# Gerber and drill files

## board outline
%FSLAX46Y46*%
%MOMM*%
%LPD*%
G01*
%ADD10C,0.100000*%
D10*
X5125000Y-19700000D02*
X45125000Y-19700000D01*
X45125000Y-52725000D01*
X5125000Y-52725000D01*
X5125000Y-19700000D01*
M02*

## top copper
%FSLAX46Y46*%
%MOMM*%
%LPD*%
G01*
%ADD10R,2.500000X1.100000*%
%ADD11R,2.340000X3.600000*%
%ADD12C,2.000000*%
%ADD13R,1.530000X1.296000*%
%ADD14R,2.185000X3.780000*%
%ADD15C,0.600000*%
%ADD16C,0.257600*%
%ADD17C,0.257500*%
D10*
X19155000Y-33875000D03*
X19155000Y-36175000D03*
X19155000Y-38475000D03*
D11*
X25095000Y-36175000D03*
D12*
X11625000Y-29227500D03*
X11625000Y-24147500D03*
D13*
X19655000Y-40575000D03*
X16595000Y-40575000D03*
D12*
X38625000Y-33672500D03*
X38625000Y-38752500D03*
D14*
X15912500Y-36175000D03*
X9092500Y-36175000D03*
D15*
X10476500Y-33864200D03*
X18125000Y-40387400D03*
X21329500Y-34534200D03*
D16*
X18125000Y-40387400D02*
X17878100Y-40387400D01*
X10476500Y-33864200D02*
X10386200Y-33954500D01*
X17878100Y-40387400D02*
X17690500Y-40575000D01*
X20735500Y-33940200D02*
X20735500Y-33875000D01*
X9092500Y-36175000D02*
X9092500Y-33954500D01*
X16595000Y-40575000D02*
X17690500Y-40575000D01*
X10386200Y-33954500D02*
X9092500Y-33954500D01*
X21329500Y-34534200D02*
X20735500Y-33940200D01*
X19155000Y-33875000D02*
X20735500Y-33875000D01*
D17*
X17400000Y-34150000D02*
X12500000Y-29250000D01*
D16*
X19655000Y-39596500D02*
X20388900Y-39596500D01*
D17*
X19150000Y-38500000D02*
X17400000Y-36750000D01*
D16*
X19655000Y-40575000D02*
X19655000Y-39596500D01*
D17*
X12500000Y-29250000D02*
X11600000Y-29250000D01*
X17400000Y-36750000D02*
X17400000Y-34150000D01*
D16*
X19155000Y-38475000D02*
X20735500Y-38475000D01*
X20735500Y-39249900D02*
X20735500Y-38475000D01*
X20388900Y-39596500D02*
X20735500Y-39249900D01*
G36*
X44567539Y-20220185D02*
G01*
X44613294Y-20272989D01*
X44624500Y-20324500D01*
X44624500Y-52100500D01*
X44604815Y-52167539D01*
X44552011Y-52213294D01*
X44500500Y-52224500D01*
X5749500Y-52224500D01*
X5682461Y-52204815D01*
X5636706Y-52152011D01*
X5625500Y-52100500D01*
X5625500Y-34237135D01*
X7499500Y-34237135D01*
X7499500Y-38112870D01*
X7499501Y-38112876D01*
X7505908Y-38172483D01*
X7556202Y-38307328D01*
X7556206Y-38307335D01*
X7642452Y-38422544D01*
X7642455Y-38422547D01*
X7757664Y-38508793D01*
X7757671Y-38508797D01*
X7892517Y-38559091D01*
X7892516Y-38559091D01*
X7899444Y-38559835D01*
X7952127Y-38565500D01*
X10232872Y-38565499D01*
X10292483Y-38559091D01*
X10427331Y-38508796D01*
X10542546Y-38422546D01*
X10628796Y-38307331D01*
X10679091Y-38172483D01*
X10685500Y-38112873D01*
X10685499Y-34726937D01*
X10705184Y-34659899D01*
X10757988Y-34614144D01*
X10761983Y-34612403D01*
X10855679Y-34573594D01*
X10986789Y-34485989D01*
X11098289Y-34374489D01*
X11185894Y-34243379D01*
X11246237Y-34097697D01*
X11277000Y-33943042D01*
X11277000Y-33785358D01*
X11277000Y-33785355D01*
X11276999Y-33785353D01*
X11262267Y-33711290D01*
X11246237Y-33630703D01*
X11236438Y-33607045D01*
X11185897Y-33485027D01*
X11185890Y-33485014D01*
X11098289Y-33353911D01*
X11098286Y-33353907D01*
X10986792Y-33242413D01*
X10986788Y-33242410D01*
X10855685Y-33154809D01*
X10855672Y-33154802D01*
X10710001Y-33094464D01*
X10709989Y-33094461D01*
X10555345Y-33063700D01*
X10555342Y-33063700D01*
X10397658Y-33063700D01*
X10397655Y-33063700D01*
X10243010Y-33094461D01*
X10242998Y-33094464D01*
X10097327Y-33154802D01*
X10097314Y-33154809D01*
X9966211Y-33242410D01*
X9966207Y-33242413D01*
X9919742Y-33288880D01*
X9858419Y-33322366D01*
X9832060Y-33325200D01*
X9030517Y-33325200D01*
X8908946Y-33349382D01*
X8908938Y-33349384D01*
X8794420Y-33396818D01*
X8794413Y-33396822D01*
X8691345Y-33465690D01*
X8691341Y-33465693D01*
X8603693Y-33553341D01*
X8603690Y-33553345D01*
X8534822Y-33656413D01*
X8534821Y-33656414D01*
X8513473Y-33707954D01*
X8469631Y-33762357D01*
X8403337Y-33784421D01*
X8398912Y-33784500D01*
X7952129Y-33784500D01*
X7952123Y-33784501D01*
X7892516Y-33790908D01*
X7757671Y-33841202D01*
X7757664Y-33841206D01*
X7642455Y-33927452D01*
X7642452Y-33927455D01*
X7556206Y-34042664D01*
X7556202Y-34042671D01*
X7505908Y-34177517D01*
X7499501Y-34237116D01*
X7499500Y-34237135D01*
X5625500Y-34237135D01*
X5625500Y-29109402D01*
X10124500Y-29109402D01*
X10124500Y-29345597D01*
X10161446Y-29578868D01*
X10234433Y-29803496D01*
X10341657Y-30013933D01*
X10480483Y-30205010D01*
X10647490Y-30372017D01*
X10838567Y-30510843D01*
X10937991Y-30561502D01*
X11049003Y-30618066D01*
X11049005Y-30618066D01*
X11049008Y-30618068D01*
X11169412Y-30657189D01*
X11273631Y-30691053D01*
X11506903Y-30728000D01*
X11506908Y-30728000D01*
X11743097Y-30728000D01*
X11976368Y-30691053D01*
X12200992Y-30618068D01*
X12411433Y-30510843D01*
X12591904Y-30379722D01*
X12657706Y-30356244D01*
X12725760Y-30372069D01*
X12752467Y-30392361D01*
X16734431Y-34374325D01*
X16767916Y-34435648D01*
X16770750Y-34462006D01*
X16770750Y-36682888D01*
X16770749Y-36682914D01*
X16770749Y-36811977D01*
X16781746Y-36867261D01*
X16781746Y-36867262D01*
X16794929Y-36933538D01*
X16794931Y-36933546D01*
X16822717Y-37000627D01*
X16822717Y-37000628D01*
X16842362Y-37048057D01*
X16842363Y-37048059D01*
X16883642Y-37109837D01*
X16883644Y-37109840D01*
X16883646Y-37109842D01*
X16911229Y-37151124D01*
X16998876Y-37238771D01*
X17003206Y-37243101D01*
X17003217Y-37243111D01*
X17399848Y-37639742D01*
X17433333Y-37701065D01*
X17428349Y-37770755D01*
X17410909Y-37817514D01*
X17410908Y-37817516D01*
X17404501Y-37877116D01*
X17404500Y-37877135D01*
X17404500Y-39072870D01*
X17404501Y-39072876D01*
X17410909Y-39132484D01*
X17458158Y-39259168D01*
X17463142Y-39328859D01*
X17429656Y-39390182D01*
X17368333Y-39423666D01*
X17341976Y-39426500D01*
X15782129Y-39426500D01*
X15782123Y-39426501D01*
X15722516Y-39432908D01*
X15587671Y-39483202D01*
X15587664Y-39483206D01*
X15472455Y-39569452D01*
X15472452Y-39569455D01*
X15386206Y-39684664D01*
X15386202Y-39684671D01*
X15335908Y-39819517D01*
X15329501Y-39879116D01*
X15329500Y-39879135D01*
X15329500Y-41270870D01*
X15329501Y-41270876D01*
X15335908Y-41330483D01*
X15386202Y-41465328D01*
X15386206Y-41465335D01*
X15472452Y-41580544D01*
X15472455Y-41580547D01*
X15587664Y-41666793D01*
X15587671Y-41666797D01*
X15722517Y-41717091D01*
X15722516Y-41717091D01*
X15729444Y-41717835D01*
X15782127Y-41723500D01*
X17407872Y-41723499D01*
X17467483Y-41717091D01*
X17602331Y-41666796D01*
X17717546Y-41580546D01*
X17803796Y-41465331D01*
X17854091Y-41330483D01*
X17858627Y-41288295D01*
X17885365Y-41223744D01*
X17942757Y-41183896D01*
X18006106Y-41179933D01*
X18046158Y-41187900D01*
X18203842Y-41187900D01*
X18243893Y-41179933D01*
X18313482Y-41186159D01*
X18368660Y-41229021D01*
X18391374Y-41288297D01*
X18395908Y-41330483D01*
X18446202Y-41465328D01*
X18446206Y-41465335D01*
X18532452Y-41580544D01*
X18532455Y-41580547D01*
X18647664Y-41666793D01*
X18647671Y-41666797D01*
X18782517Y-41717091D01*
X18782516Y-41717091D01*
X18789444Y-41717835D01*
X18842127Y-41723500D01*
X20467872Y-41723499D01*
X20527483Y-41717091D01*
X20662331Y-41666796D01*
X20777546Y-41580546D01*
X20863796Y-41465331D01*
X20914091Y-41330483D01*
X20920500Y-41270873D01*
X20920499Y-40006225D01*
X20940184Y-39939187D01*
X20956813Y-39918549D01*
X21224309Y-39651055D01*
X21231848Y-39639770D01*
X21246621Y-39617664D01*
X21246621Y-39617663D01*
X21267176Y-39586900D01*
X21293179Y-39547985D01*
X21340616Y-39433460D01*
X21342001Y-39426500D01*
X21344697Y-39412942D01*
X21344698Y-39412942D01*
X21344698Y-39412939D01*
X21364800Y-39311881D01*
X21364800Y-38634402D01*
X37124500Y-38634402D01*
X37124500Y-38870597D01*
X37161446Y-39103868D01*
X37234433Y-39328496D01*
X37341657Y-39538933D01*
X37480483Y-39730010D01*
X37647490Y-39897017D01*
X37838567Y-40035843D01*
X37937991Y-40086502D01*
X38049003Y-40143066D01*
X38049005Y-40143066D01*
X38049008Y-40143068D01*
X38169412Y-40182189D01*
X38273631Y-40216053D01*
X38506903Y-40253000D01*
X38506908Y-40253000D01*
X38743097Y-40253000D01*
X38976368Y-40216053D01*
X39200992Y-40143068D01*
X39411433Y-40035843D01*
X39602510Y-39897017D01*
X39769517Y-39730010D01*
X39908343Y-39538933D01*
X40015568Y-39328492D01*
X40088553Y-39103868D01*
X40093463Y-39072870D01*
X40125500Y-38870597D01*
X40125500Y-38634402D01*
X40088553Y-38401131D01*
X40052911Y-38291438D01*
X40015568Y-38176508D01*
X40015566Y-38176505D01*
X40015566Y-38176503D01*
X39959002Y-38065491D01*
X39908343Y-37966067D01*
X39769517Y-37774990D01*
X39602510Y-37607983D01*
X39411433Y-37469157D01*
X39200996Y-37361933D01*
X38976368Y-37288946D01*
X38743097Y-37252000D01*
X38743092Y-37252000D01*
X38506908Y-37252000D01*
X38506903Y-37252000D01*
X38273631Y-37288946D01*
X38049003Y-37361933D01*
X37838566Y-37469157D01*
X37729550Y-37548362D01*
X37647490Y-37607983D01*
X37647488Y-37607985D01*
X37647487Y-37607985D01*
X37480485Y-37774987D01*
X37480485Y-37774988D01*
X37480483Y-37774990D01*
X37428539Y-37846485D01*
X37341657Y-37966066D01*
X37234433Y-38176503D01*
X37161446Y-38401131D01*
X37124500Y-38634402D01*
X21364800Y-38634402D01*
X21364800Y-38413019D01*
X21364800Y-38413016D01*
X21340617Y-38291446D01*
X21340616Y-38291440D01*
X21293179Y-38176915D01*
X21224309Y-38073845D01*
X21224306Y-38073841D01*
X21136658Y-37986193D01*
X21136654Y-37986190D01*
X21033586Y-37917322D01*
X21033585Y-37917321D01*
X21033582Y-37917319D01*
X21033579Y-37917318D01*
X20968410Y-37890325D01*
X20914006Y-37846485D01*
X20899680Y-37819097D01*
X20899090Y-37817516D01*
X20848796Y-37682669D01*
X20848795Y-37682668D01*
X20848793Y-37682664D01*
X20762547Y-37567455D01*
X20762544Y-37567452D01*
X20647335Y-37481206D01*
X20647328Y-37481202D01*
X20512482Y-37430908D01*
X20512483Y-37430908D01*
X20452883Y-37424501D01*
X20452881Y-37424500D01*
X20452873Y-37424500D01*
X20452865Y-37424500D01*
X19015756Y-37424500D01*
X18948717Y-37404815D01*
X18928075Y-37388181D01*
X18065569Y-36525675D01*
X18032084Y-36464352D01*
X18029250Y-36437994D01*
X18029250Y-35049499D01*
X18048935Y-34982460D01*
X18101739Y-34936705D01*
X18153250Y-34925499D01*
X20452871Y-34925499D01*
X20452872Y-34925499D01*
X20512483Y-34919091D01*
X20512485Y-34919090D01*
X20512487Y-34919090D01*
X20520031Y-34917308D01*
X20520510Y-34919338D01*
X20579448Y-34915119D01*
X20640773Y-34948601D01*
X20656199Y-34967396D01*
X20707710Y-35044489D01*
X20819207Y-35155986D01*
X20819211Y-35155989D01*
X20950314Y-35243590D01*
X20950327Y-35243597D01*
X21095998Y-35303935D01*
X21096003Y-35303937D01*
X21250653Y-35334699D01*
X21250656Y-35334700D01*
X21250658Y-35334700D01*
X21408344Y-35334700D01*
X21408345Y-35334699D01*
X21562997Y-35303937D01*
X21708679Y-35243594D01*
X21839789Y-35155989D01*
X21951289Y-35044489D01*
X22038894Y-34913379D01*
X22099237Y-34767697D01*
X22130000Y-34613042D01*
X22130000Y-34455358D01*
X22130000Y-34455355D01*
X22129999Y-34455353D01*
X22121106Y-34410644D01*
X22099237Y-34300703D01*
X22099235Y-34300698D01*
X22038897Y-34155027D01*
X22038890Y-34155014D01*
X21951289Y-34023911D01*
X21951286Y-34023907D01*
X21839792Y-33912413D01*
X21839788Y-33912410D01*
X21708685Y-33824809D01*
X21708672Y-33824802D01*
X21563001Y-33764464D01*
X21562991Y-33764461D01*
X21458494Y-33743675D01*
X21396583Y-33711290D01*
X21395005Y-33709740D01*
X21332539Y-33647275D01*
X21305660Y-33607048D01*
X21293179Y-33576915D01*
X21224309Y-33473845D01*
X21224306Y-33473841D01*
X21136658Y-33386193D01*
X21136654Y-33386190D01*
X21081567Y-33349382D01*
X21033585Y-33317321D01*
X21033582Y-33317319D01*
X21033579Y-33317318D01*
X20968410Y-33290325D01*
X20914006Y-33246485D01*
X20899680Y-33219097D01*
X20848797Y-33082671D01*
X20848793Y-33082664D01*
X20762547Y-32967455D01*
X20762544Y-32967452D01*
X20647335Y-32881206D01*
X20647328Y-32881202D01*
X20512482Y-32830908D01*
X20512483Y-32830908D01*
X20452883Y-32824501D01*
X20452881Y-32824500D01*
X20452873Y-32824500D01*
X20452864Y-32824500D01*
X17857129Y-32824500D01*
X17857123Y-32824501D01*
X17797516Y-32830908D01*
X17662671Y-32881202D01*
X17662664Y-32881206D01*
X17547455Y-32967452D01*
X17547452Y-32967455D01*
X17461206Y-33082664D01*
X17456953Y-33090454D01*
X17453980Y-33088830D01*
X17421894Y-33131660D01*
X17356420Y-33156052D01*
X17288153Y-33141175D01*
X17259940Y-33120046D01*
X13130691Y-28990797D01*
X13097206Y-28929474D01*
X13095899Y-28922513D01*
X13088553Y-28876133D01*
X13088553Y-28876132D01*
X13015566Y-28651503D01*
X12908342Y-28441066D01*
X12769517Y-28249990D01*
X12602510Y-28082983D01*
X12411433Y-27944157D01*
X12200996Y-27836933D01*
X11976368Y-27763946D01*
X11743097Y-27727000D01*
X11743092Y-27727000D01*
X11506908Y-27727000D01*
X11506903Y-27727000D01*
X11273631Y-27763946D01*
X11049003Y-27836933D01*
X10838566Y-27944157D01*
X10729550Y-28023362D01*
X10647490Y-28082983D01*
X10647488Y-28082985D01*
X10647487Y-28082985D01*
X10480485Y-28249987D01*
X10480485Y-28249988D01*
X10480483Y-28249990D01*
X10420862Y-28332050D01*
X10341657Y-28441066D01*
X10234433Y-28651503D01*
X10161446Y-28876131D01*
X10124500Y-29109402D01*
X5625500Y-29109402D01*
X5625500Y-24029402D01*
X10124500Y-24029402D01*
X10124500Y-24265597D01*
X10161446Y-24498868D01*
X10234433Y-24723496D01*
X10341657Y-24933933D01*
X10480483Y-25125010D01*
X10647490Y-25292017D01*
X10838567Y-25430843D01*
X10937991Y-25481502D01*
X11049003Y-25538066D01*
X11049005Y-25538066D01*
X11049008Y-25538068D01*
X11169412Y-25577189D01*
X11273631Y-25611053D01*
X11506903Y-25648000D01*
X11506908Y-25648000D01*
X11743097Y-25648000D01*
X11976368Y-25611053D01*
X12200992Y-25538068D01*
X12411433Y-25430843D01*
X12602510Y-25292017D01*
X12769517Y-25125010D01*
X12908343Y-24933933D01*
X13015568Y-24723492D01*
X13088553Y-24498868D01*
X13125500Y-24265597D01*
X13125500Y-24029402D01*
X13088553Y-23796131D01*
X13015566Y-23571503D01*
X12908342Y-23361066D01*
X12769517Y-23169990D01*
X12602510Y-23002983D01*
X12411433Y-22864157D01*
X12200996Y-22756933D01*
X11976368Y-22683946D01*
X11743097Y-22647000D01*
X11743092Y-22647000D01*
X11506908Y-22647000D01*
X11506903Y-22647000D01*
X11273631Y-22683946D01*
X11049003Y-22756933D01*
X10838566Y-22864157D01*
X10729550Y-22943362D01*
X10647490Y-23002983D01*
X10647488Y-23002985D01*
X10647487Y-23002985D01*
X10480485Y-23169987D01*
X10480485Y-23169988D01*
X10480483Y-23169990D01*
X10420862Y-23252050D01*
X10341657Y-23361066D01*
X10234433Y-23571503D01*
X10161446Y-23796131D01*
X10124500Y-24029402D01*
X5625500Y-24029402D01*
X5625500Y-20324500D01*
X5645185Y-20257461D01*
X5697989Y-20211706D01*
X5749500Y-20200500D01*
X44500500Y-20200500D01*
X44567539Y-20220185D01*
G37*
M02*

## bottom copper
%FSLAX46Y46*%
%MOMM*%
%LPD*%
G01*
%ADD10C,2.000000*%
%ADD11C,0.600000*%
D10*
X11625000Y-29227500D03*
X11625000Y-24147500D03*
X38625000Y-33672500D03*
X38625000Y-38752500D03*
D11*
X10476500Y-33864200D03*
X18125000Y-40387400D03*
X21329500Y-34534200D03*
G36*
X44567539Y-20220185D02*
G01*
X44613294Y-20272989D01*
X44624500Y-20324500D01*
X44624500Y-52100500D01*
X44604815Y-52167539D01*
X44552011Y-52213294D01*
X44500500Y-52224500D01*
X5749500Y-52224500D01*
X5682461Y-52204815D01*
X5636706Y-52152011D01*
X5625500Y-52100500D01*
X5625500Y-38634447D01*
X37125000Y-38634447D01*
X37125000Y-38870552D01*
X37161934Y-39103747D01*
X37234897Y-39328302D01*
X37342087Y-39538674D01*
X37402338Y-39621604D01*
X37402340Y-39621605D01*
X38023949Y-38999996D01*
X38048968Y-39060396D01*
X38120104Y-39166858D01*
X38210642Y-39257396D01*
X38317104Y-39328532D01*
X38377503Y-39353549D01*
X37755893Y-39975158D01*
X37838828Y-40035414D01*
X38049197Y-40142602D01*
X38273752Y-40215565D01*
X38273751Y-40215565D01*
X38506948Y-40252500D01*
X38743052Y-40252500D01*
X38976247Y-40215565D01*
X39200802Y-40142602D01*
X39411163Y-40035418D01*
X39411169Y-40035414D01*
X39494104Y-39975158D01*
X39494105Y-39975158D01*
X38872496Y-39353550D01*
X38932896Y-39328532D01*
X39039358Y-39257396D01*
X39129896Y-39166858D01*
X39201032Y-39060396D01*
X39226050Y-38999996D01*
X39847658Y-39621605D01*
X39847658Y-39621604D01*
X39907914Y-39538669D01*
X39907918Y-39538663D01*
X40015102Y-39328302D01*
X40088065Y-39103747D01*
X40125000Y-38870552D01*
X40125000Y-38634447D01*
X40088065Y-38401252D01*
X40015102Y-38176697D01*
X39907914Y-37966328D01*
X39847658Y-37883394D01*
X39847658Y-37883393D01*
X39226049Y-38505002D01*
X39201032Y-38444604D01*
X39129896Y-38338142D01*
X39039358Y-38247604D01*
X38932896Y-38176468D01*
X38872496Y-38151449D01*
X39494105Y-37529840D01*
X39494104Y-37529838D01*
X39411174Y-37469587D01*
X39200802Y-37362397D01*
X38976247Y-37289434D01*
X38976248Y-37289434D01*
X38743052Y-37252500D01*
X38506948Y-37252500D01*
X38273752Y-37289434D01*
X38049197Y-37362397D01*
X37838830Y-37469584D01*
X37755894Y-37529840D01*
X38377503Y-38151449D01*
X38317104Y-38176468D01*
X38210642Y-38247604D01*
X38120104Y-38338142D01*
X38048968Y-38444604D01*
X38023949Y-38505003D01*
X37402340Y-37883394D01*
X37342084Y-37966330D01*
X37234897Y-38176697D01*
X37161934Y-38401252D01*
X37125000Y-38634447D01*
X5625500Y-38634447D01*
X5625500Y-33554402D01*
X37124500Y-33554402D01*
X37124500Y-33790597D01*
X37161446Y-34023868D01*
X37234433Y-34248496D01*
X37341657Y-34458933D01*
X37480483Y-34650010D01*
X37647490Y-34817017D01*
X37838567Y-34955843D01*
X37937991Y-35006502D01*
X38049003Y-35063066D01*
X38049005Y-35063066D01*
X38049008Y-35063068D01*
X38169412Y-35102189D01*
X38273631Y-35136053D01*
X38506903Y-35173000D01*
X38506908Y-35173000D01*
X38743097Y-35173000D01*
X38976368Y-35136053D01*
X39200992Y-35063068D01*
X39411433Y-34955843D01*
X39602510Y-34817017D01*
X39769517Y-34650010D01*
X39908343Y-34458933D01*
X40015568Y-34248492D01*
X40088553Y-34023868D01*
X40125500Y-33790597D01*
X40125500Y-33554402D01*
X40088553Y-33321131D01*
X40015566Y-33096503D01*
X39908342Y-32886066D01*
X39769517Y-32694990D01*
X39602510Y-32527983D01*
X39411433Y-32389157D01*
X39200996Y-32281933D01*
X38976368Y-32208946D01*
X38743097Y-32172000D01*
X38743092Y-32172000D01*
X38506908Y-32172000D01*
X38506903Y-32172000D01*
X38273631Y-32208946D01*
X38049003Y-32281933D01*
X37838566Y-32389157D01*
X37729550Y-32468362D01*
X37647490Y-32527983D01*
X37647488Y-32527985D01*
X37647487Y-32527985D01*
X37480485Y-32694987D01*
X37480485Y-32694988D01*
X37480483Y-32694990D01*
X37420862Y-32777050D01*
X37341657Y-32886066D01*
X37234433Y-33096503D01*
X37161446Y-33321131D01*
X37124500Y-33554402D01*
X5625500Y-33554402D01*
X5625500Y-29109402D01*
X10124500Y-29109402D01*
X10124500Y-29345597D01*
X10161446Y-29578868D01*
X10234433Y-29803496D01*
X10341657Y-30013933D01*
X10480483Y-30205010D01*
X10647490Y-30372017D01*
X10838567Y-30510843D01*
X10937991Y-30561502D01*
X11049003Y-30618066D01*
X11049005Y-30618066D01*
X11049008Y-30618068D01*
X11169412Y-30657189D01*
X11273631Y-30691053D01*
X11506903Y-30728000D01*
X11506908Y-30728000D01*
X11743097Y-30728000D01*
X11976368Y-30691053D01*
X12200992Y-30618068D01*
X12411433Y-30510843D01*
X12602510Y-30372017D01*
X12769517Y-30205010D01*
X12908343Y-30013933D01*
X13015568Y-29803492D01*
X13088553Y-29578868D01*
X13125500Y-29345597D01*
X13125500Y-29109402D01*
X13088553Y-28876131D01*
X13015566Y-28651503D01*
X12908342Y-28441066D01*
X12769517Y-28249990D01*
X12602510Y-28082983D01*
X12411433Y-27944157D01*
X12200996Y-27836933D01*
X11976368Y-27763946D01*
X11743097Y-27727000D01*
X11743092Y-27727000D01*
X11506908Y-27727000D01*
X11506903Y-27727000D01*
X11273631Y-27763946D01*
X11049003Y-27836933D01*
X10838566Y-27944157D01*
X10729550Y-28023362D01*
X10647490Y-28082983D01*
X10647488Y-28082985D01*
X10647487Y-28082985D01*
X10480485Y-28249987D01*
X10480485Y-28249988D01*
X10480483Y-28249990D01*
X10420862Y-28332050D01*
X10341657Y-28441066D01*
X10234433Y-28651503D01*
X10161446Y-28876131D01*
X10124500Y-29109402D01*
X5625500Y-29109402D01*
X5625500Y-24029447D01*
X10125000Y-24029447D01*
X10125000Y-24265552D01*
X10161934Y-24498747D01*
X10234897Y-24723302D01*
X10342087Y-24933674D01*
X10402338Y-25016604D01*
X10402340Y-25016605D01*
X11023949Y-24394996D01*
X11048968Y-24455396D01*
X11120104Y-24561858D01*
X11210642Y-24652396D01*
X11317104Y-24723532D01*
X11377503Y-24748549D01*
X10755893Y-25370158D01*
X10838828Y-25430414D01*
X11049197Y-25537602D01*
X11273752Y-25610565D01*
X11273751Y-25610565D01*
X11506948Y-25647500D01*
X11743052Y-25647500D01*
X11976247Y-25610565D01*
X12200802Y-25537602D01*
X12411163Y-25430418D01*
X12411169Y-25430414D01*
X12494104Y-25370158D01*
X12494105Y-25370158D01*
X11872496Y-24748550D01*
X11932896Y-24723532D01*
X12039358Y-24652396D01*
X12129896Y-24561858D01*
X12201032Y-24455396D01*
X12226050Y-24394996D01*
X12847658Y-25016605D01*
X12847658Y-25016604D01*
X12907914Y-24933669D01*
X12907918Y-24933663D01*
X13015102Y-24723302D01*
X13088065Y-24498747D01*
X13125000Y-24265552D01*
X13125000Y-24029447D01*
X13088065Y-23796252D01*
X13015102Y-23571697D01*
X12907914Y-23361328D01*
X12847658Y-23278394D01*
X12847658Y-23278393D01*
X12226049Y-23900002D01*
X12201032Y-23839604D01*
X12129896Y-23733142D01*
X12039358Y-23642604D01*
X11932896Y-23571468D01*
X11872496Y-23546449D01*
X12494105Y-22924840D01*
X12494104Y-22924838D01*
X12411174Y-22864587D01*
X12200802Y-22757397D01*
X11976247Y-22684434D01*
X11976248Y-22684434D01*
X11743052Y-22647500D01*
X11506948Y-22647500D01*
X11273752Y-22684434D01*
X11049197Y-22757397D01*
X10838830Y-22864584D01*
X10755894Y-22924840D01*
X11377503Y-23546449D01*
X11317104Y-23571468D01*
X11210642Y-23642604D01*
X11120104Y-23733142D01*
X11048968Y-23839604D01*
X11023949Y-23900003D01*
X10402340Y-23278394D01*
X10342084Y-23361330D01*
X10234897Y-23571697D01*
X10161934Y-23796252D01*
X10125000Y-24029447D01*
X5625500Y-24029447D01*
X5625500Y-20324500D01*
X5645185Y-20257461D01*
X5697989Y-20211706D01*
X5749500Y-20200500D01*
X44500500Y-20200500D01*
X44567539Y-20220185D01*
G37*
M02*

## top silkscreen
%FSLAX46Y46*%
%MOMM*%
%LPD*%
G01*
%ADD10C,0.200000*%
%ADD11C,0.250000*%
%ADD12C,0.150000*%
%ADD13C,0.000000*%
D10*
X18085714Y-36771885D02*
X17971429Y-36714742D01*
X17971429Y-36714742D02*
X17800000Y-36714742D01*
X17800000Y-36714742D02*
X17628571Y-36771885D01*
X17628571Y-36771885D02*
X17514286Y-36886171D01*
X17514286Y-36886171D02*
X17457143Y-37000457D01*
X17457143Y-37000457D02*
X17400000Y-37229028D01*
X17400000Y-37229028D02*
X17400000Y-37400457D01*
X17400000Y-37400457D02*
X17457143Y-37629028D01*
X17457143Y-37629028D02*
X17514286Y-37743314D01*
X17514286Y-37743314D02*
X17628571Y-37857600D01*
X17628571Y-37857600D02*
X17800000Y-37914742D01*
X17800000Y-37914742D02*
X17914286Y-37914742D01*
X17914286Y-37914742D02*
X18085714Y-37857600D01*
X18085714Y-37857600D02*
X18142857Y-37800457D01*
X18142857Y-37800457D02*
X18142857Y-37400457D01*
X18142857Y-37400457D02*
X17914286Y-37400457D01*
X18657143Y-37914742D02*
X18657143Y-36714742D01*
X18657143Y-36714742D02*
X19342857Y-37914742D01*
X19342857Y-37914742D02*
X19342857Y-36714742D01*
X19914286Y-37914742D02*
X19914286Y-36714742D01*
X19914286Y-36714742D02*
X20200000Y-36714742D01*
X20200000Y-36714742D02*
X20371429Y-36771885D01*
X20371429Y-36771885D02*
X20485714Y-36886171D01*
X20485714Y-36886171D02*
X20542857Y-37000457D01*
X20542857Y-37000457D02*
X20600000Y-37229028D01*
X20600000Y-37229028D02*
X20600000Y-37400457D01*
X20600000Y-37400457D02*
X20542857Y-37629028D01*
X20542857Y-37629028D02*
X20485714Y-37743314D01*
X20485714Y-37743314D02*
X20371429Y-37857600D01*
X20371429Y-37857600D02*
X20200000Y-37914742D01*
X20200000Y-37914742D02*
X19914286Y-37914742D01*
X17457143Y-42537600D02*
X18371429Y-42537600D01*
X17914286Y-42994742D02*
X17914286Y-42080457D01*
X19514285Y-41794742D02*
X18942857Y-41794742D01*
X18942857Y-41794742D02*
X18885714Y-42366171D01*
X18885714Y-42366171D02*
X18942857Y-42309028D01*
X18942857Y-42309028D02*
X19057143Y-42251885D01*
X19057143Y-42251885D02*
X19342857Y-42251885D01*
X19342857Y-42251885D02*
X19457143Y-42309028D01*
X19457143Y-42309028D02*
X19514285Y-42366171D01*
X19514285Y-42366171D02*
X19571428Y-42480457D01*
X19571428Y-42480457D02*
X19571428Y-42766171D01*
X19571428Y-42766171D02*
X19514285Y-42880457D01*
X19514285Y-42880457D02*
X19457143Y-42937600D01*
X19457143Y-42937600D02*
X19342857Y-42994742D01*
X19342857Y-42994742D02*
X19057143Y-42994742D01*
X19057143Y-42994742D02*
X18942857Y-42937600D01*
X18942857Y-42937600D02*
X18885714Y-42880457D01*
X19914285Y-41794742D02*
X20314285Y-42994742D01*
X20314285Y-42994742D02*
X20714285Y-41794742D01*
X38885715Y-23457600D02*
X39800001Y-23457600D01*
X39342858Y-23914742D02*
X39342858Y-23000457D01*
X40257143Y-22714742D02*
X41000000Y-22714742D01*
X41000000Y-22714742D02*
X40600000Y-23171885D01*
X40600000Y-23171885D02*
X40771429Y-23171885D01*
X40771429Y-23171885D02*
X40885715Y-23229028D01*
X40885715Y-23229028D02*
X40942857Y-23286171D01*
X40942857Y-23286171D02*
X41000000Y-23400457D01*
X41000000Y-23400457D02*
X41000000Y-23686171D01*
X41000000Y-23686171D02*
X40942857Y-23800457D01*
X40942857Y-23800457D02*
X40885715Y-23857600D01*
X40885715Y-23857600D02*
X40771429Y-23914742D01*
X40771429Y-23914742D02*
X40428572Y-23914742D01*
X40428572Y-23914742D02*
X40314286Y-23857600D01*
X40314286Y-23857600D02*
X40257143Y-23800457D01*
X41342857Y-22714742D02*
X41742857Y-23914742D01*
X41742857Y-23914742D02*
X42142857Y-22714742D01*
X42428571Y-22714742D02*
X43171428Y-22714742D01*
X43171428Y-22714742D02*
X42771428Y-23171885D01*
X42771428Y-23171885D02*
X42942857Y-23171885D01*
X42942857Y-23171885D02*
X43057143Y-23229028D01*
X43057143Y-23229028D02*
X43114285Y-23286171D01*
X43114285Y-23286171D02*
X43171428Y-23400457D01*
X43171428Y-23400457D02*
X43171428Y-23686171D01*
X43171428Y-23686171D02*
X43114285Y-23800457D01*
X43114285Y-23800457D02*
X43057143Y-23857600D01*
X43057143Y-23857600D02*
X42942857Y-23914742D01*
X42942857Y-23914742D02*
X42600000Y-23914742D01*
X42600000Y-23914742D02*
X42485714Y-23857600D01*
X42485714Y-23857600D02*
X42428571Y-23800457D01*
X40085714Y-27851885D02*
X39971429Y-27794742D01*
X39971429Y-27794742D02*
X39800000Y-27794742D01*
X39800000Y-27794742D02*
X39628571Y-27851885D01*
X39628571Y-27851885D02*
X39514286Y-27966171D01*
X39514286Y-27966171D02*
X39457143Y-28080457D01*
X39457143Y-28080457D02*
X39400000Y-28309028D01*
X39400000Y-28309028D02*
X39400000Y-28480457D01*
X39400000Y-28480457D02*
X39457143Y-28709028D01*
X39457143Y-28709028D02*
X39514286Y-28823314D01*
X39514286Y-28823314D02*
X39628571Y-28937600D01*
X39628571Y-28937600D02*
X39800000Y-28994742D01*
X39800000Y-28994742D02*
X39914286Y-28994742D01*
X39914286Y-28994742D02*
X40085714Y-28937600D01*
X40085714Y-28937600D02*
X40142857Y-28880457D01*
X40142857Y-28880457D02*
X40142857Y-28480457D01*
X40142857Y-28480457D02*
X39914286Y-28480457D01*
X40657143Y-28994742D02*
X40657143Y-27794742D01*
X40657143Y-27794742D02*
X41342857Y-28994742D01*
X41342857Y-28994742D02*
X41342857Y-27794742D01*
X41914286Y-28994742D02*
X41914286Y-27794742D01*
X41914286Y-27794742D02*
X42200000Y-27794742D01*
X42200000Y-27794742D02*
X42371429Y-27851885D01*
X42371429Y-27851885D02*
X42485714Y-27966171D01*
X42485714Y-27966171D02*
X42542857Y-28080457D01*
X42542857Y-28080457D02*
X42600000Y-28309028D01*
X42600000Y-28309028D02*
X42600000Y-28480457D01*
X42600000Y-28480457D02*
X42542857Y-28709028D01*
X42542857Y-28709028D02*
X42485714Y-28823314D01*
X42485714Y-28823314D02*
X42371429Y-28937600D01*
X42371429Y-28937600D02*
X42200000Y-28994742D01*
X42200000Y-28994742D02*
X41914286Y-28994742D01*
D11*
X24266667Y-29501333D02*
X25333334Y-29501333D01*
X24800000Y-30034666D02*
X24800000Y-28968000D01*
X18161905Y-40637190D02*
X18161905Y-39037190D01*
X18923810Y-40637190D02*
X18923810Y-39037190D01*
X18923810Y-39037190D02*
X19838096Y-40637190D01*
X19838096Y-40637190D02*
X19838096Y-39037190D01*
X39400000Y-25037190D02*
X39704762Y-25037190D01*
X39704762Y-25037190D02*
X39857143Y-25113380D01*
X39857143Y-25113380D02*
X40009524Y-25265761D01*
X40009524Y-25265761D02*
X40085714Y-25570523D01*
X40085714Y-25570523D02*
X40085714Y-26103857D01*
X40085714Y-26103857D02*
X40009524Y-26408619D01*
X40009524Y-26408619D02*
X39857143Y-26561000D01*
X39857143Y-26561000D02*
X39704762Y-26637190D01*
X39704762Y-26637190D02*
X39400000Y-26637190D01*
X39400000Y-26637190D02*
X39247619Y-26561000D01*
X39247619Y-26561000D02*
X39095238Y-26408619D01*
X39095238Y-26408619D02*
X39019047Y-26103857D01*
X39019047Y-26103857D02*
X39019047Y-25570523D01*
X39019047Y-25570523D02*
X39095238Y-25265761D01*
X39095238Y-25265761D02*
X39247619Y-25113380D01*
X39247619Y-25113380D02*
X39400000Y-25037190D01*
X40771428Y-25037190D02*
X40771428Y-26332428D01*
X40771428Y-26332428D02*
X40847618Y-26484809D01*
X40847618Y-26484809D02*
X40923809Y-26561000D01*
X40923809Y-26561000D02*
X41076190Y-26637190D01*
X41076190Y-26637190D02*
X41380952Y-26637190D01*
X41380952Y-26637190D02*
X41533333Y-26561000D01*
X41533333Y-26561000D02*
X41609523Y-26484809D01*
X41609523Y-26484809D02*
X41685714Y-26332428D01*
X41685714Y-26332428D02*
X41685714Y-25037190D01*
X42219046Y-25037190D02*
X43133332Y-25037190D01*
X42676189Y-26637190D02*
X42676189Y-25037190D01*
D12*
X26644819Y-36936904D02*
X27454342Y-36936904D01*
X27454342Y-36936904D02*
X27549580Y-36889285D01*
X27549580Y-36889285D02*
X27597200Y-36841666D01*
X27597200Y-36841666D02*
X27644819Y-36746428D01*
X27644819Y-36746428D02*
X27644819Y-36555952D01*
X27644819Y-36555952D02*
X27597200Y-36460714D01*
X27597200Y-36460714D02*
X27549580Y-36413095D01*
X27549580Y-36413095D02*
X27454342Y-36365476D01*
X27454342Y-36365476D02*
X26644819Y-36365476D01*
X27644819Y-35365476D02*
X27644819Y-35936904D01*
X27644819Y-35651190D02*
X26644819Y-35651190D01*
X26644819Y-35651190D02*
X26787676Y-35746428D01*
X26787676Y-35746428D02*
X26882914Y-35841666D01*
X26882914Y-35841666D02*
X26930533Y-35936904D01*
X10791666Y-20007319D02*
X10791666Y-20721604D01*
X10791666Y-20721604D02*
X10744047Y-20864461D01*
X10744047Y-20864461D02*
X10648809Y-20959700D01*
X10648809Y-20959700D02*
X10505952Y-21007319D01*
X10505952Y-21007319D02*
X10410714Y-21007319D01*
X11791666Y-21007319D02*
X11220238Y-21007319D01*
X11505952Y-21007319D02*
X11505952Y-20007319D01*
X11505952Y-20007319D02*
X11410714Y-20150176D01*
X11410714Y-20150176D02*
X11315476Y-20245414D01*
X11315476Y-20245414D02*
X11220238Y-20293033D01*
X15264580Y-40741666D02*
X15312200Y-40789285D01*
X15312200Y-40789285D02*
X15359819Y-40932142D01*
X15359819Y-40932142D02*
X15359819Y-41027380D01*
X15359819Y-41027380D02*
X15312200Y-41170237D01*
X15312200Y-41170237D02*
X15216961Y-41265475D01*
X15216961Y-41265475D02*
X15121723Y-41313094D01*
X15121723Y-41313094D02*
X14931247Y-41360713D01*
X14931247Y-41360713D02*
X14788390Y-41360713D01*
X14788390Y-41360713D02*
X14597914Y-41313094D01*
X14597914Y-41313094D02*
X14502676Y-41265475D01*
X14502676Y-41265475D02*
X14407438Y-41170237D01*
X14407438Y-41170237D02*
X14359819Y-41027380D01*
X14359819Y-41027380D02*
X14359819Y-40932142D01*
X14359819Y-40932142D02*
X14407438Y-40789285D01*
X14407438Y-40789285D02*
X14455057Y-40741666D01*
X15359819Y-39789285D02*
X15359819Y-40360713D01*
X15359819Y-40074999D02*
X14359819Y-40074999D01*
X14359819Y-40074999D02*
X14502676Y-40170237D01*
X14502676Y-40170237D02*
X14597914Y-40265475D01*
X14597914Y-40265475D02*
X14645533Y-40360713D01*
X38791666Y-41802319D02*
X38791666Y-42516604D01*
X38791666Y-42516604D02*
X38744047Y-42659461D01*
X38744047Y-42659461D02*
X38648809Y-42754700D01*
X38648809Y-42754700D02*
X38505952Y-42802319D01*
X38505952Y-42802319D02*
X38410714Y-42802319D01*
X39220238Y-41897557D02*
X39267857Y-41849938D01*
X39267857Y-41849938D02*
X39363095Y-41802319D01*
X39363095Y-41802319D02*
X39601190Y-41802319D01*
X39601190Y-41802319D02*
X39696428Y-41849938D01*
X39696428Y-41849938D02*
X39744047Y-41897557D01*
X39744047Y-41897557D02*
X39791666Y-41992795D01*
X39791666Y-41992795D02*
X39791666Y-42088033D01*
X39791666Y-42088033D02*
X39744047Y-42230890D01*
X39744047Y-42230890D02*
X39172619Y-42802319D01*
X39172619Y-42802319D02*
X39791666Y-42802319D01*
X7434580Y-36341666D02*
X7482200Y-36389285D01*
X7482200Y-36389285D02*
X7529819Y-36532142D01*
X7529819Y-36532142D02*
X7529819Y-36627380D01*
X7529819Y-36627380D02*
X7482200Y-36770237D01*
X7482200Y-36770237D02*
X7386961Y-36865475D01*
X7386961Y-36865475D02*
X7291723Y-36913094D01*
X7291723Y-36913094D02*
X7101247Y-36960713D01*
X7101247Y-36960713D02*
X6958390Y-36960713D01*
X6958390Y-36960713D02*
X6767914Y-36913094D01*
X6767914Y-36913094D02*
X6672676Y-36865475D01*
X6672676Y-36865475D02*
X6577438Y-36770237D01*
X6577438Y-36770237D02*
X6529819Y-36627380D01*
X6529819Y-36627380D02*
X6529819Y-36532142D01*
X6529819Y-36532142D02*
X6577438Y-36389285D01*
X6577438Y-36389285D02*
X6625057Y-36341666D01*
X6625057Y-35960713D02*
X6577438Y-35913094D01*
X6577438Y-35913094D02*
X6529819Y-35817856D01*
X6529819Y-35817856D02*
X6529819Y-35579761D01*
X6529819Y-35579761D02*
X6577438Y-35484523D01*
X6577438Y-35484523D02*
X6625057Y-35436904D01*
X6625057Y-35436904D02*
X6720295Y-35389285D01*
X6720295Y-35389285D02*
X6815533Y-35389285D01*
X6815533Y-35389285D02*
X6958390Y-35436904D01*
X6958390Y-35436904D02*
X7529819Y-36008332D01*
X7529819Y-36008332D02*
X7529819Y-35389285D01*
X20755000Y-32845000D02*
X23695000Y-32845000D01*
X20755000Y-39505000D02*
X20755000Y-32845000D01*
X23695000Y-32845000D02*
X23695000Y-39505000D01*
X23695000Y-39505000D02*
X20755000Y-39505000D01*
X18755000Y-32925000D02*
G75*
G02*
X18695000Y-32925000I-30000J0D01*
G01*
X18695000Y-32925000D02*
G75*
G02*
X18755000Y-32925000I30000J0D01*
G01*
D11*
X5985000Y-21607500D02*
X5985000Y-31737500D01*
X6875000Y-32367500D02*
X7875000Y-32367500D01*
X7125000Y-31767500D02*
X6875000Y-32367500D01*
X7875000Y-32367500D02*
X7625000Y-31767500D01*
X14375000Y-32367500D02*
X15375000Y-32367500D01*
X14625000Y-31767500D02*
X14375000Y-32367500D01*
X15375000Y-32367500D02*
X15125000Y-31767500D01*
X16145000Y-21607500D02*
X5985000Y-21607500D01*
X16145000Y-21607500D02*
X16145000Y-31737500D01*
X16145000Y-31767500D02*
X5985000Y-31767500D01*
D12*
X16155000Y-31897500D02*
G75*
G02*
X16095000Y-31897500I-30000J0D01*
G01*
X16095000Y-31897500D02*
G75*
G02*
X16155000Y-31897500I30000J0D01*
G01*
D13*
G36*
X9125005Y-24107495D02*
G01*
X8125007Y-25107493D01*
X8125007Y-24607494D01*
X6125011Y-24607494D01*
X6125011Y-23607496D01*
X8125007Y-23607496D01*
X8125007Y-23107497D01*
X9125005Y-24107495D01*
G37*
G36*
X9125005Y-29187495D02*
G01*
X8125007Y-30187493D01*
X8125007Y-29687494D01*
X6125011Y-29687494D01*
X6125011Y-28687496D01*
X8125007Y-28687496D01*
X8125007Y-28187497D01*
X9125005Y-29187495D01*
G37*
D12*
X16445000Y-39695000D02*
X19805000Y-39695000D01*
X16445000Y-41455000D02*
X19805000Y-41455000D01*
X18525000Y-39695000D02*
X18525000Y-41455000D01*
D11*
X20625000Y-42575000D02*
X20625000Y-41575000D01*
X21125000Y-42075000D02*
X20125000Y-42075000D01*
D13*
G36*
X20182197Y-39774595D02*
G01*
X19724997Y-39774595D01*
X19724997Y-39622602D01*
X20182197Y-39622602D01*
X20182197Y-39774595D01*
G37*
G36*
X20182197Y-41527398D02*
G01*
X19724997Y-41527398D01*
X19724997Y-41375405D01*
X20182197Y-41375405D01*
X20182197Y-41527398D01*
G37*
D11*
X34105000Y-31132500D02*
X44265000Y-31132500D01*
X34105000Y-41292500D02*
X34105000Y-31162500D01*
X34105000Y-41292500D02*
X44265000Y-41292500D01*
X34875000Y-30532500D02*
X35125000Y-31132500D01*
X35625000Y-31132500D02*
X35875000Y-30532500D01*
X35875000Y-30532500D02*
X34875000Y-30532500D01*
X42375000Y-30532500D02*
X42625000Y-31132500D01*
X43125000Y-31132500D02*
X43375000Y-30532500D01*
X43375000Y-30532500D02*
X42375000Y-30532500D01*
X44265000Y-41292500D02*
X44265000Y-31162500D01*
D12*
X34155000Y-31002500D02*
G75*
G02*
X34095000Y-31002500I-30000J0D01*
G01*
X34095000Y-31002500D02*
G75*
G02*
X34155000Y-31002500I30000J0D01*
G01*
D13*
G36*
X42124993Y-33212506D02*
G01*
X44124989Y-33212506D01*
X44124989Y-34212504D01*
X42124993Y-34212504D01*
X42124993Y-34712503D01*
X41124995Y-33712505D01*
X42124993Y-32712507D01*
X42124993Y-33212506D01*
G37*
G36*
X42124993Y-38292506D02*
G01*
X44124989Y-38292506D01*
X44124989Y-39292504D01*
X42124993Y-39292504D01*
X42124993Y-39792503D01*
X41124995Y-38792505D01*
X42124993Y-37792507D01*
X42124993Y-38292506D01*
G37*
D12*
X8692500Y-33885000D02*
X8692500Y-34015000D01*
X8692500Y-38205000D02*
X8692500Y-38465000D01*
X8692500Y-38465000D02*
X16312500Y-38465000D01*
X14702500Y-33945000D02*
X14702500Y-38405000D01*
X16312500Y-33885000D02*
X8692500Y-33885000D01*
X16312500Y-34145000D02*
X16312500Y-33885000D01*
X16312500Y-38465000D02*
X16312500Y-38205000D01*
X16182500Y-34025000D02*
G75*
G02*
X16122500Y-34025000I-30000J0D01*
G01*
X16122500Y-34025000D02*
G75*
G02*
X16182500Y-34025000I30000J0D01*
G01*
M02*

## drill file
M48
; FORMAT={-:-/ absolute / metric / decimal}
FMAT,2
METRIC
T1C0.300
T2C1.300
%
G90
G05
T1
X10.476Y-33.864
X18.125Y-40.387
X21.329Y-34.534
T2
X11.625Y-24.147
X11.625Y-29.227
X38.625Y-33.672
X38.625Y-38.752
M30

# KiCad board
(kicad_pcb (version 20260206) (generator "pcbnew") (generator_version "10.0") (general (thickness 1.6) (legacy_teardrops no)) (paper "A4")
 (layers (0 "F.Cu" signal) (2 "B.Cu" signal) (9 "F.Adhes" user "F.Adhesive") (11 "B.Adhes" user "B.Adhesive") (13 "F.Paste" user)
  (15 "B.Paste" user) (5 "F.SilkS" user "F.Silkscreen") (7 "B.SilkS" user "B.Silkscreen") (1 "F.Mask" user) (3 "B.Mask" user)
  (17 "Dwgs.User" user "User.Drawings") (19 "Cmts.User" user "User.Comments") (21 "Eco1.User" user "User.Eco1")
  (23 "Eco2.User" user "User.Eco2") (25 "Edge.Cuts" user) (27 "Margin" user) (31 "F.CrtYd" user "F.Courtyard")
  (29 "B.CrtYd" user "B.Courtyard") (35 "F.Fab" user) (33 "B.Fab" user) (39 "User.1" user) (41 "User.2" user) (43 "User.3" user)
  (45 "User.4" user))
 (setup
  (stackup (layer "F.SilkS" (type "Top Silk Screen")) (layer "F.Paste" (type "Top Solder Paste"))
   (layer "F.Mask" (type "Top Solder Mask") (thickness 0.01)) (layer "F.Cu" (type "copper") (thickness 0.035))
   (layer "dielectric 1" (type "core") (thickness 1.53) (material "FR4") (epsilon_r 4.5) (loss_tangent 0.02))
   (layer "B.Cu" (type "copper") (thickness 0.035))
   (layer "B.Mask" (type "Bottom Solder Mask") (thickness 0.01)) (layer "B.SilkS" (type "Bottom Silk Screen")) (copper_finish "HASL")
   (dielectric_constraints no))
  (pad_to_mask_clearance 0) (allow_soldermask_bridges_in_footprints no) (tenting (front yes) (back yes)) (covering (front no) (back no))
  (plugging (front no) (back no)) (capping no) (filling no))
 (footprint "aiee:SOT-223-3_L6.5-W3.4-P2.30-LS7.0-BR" (layer "F.Cu") (at 22.125 36.175 180)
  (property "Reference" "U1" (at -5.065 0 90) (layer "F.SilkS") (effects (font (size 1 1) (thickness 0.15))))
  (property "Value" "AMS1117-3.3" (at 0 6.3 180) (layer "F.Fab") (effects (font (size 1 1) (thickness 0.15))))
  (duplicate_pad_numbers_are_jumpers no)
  (fp_line (start 1.37 3.33) (end -1.57 3.33) (stroke (width 0.15) (type solid)) (layer "F.SilkS"))
  (fp_line (start 1.37 -3.33) (end 1.37 3.33) (stroke (width 0.15) (type solid)) (layer "F.SilkS"))
  (fp_line (start -1.57 3.33) (end -1.57 -3.33) (stroke (width 0.15) (type solid)) (layer "F.SilkS"))
  (fp_line (start -1.57 -3.33) (end 1.37 -3.33) (stroke (width 0.15) (type solid)) (layer "F.SilkS"))
  (fp_circle (center 3.4 3.25) (end 3.43 3.25) (stroke (width 0.15) (type solid)) (fill no) (layer "F.SilkS"))
  (pad "1" smd rect (at 2.97 2.3 180) (size 2.5 1.1) (layers "F.Cu" "F.Mask" "F.Paste") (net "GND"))
  (pad "2" smd rect (at 2.97 0 180) (size 2.5 1.1) (layers "F.Cu" "F.Mask" "F.Paste") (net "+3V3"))
  (pad "3" smd rect (at 2.97 -2.3 180) (size 2.5 1.1) (layers "F.Cu" "F.Mask" "F.Paste") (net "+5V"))
  (pad "4" smd rect (at -2.97 0 180) (size 2.34 3.6) (layers "F.Cu" "F.Mask" "F.Paste") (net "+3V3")))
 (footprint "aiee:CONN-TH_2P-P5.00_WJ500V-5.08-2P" (layer "F.Cu") (at 11.625 26.6875 90)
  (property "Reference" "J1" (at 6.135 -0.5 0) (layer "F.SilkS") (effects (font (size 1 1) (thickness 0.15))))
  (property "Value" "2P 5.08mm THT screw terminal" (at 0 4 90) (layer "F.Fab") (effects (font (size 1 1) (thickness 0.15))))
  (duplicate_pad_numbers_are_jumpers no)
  (fp_line (start 5.08 -5.64) (end -5.05 -5.64) (stroke (width 0.25) (type solid)) (layer "F.SilkS"))
  (fp_line (start -5.68 -4.75) (end -5.68 -3.75) (stroke (width 0.25) (type solid)) (layer "F.SilkS"))
  (fp_line (start -5.08 -4.5) (end -5.68 -4.75) (stroke (width 0.25) (type solid)) (layer "F.SilkS"))
  (fp_line (start -5.68 -3.75) (end -5.08 -4) (stroke (width 0.25) (type solid)) (layer "F.SilkS"))
  (fp_line (start -5.68 2.75) (end -5.68 3.75) (stroke (width 0.25) (type solid)) (layer "F.SilkS"))
  (fp_line (start -5.08 3) (end -5.68 2.75) (stroke (width 0.25) (type solid)) (layer "F.SilkS"))
  (fp_line (start -5.68 3.75) (end -5.08 3.5) (stroke (width 0.25) (type solid)) (layer "F.SilkS"))
  (fp_line (start 5.08 4.52) (end 5.08 -5.64) (stroke (width 0.25) (type solid)) (layer "F.SilkS"))
  (fp_line (start 5.08 4.52) (end -5.05 4.52) (stroke (width 0.25) (type solid)) (layer "F.SilkS"))
  (fp_line (start -5.08 4.52) (end -5.08 -5.64) (stroke (width 0.25) (type solid)) (layer "F.SilkS"))
  (fp_circle (center -5.21 4.5) (end -5.18 4.5) (stroke (width 0.15) (type solid)) (fill no) (layer "F.SilkS"))
  (fp_poly
   (pts (xy 2.080006 -5.499989) (xy 3.080004 -5.499989) (xy 3.080004 -3.499993) (xy 3.580003 -3.499993) (xy 2.580005 -2.499995)
    (xy 1.580007 -3.499993) (xy 2.080006 -3.499993) (xy 2.080006 -5.499989))
   (stroke (width 0) (type solid)) (fill yes) (layer "F.SilkS"))
  (fp_poly
   (pts (xy -2.999994 -5.499989) (xy -1.999996 -5.499989) (xy -1.999996 -3.499993) (xy -1.499997 -3.499993) (xy -2.499995 -2.499995)
    (xy -3.499993 -3.499993) (xy -2.999994 -3.499993) (xy -2.999994 -5.499989))
   (stroke (width 0) (type solid)) (fill yes) (layer "F.SilkS"))
  (pad "1" thru_hole circle (at -2.54 0 270) (size 2 2) (drill 1.300022) (layers "*.Cu" "*.Mask") (remove_unused_layers no) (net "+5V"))
  (pad "2" thru_hole circle (at 2.54 0 270) (size 2 2) (drill 1.300022) (layers "*.Cu" "*.Mask") (remove_unused_layers no) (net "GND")))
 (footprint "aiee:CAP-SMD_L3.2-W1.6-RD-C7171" (layer "F.Cu") (at 18.125 40.575 180)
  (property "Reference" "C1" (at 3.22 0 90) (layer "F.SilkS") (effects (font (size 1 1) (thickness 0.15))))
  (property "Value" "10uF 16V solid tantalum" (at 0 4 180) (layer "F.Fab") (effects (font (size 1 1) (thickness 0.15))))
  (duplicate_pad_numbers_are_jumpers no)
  (fp_line (start 1.68 0.88) (end -1.68 0.88) (stroke (width 0.15) (type solid)) (layer "F.SilkS"))
  (fp_line (start 1.68 -0.88) (end -1.68 -0.88) (stroke (width 0.15) (type solid)) (layer "F.SilkS"))
  (fp_line (start -0.4 0.88) (end -0.4 -0.88) (stroke (width 0.15) (type solid)) (layer "F.SilkS"))
  (fp_line (start -2.5 -2) (end -2.5 -1) (stroke (width 0.25) (type solid)) (layer "F.SilkS"))
  (fp_line (start -3 -1.5) (end -2 -1.5) (stroke (width 0.25) (type solid)) (layer "F.SilkS"))
  (fp_poly
   (pts (xy -1.599997 0.952398) (xy -1.599997 0.800405) (xy -2.057197 0.800405) (xy -2.057197 0.952398) (xy -1.599997 0.952398))
   (stroke (width 0) (type solid)) (fill yes) (layer "F.SilkS"))
  (fp_poly
   (pts (xy -1.599997 -0.952398) (xy -1.599997 -0.800405) (xy -2.057197 -0.800405) (xy -2.057197 -0.952398) (xy -1.599997 -0.952398))
   (stroke (width 0) (type solid)) (fill yes) (layer "F.SilkS"))
  (pad "1" smd rect (at -1.53 0) (size 1.53 1.296) (layers "F.Cu" "F.Mask" "F.Paste") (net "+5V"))
  (pad "2" smd rect (at 1.53 0) (size 1.53 1.296) (layers "F.Cu" "F.Mask" "F.Paste") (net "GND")))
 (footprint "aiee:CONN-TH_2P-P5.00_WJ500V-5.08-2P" (layer "F.Cu") (at 38.625 36.2125 -90)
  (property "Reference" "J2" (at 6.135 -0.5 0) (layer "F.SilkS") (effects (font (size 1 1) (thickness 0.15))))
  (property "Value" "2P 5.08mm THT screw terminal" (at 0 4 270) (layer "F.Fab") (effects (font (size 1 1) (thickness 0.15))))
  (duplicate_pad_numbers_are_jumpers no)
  (fp_line (start -5.08 4.52) (end -5.08 -5.64) (stroke (width 0.25) (type solid)) (layer "F.SilkS"))
  (fp_line (start 5.08 4.52) (end -5.05 4.52) (stroke (width 0.25) (type solid)) (layer "F.SilkS"))
  (fp_line (start 5.08 4.52) (end 5.08 -5.64) (stroke (width 0.25) (type solid)) (layer "F.SilkS"))
  (fp_line (start -5.68 3.75) (end -5.08 3.5) (stroke (width 0.25) (type solid)) (layer "F.SilkS"))
  (fp_line (start -5.08 3) (end -5.68 2.75) (stroke (width 0.25) (type solid)) (layer "F.SilkS"))
  (fp_line (start -5.68 2.75) (end -5.68 3.75) (stroke (width 0.25) (type solid)) (layer "F.SilkS"))
  (fp_line (start -5.68 -3.75) (end -5.08 -4) (stroke (width 0.25) (type solid)) (layer "F.SilkS"))
  (fp_line (start -5.08 -4.5) (end -5.68 -4.75) (stroke (width 0.25) (type solid)) (layer "F.SilkS"))
  (fp_line (start -5.68 -4.75) (end -5.68 -3.75) (stroke (width 0.25) (type solid)) (layer "F.SilkS"))
  (fp_line (start 5.08 -5.64) (end -5.05 -5.64) (stroke (width 0.25) (type solid)) (layer "F.SilkS"))
  (fp_circle (center -5.21 4.5) (end -5.18 4.5) (stroke (width 0.15) (type solid)) (fill no) (layer "F.SilkS"))
  (fp_poly
   (pts (xy -2.999994 -5.499989) (xy -1.999996 -5.499989) (xy -1.999996 -3.499993) (xy -1.499997 -3.499993) (xy -2.499995 -2.499995)
    (xy -3.499993 -3.499993) (xy -2.999994 -3.499993) (xy -2.999994 -5.499989))
   (stroke (width 0) (type solid)) (fill yes) (layer "F.SilkS"))
  (fp_poly
   (pts (xy 2.080006 -5.499989) (xy 3.080004 -5.499989) (xy 3.080004 -3.499993) (xy 3.580003 -3.499993) (xy 2.580005 -2.499995)
    (xy 1.580007 -3.499993) (xy 2.080006 -3.499993) (xy 2.080006 -5.499989))
   (stroke (width 0) (type solid)) (fill yes) (layer "F.SilkS"))
  (pad "1" thru_hole circle (at -2.54 0 90) (size 2 2) (drill 1.300022) (layers "*.Cu" "*.Mask") (remove_unused_layers no) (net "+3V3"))
  (pad "2" thru_hole circle (at 2.54 0 90) (size 2 2) (drill 1.300022) (layers "*.Cu" "*.Mask") (remove_unused_layers no) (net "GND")))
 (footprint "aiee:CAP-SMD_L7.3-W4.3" (layer "F.Cu") (at 12.5025 36.175)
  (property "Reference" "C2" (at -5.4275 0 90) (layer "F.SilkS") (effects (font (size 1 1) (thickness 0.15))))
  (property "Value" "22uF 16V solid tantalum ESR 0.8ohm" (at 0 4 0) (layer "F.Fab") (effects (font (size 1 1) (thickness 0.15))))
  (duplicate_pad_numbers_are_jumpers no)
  (fp_line (start -3.81 -2.29) (end -3.81 -2.16) (stroke (width 0.15) (type solid)) (layer "F.SilkS"))
  (fp_line (start -3.81 2.03) (end -3.81 2.29) (stroke (width 0.15) (type solid)) (layer "F.SilkS"))
  (fp_line (start -3.81 2.29) (end 3.81 2.29) (stroke (width 0.15) (type solid)) (layer "F.SilkS"))
  (fp_line (start 2.2 -2.23) (end 2.2 2.23) (stroke (width 0.15) (type solid)) (layer "F.SilkS"))
  (fp_line (start 3.81 -2.29) (end -3.81 -2.29) (stroke (width 0.15) (type solid)) (layer "F.SilkS"))
  (fp_line (start 3.81 -2.03) (end 3.81 -2.29) (stroke (width 0.15) (type solid)) (layer "F.SilkS"))
  (fp_line (start 3.81 2.29) (end 3.81 2.03) (stroke (width 0.15) (type solid)) (layer "F.SilkS"))
  (fp_circle (center 3.65 -2.15) (end 3.68 -2.15) (stroke (width 0.15) (type solid)) (fill no) (layer "F.SilkS"))
  (pad "1" smd rect (at 3.41 0 180) (size 2.185 3.78) (layers "F.Cu" "F.Mask" "F.Paste") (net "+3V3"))
  (pad "2" smd rect (at -3.41 0 180) (size 2.185 3.78) (layers "F.Cu" "F.Mask" "F.Paste") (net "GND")))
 (gr_rect (start 5.125 19.7) (end 45.125 52.725) (stroke (width 0.1) (type default)) (fill no) (layer "Edge.Cuts"))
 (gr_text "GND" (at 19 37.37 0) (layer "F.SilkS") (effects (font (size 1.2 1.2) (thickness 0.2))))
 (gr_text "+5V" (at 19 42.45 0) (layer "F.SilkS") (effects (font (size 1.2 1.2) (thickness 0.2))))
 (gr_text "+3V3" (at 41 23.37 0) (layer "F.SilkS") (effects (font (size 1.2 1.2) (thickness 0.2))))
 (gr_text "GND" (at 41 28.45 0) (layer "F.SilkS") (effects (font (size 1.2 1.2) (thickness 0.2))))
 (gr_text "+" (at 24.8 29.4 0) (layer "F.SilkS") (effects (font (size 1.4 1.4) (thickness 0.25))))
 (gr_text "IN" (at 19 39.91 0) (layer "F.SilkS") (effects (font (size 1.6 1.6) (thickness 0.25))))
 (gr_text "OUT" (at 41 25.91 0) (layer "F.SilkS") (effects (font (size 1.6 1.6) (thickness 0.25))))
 (segment (start 18.125 40.3874) (end 17.8781 40.3874) (width 0.2576) (layer "F.Cu") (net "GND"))
 (segment (start 10.4765 33.8642) (end 10.3862 33.9545) (width 0.2576) (layer "F.Cu") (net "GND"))
 (segment (start 17.8781 40.3874) (end 17.6905 40.575) (width 0.2576) (layer "F.Cu") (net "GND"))
 (segment (start 20.7355 33.9402) (end 20.7355 33.875) (width 0.2576) (layer "F.Cu") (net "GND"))
 (segment (start 9.0925 36.175) (end 9.0925 33.9545) (width 0.2576) (layer "F.Cu") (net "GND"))
 (segment (start 16.595 40.575) (end 17.6905 40.575) (width 0.2576) (layer "F.Cu") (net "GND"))
 (segment (start 10.3862 33.9545) (end 9.0925 33.9545) (width 0.2576) (layer "F.Cu") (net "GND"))
 (segment (start 21.3295 34.5342) (end 20.7355 33.9402) (width 0.2576) (layer "F.Cu") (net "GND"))
 (segment (start 19.155 33.875) (end 20.7355 33.875) (width 0.2576) (layer "F.Cu") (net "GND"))
 (via (at 10.4765 33.8642) (size 0.6) (drill 0.3) (layers "F.Cu" "B.Cu") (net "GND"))
 (via (at 18.125 40.3874) (size 0.6) (drill 0.3) (layers "F.Cu" "B.Cu") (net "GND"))
 (via (at 21.3295 34.5342) (size 0.6) (drill 0.3) (layers "F.Cu" "B.Cu") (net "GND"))
 (segment (start 17.4 34.15) (end 12.5 29.25) (width 0.2575) (layer "F.Cu") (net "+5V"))
 (segment (start 19.655 39.5965) (end 20.3889 39.5965) (width 0.2576) (layer "F.Cu") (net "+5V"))
 (segment (start 19.15 38.5) (end 17.4 36.75) (width 0.2575) (layer "F.Cu") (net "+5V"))
 (segment (start 19.655 40.575) (end 19.655 39.5965) (width 0.2576) (layer "F.Cu") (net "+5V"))
 (segment (start 12.5 29.25) (end 11.6 29.25) (width 0.2575) (layer "F.Cu") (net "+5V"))
 (segment (start 17.4 36.75) (end 17.4 34.15) (width 0.2575) (layer "F.Cu") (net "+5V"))
 (segment (start 19.155 38.475) (end 20.7355 38.475) (width 0.2576) (layer "F.Cu") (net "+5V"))
 (segment (start 20.7355 39.2499) (end 20.7355 38.475) (width 0.2576) (layer "F.Cu") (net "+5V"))
 (segment (start 20.3889 39.5965) (end 20.7355 39.2499) (width 0.2576) (layer "F.Cu") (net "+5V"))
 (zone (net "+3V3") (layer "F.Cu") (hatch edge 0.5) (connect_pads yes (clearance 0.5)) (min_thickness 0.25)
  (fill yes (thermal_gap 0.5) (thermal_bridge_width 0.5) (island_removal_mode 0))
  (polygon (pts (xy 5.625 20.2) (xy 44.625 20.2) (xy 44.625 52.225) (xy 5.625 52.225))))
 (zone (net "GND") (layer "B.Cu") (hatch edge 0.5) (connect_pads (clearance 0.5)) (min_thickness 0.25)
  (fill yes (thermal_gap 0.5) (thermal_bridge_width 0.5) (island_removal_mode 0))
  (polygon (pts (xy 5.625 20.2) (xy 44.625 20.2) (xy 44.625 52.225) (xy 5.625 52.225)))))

